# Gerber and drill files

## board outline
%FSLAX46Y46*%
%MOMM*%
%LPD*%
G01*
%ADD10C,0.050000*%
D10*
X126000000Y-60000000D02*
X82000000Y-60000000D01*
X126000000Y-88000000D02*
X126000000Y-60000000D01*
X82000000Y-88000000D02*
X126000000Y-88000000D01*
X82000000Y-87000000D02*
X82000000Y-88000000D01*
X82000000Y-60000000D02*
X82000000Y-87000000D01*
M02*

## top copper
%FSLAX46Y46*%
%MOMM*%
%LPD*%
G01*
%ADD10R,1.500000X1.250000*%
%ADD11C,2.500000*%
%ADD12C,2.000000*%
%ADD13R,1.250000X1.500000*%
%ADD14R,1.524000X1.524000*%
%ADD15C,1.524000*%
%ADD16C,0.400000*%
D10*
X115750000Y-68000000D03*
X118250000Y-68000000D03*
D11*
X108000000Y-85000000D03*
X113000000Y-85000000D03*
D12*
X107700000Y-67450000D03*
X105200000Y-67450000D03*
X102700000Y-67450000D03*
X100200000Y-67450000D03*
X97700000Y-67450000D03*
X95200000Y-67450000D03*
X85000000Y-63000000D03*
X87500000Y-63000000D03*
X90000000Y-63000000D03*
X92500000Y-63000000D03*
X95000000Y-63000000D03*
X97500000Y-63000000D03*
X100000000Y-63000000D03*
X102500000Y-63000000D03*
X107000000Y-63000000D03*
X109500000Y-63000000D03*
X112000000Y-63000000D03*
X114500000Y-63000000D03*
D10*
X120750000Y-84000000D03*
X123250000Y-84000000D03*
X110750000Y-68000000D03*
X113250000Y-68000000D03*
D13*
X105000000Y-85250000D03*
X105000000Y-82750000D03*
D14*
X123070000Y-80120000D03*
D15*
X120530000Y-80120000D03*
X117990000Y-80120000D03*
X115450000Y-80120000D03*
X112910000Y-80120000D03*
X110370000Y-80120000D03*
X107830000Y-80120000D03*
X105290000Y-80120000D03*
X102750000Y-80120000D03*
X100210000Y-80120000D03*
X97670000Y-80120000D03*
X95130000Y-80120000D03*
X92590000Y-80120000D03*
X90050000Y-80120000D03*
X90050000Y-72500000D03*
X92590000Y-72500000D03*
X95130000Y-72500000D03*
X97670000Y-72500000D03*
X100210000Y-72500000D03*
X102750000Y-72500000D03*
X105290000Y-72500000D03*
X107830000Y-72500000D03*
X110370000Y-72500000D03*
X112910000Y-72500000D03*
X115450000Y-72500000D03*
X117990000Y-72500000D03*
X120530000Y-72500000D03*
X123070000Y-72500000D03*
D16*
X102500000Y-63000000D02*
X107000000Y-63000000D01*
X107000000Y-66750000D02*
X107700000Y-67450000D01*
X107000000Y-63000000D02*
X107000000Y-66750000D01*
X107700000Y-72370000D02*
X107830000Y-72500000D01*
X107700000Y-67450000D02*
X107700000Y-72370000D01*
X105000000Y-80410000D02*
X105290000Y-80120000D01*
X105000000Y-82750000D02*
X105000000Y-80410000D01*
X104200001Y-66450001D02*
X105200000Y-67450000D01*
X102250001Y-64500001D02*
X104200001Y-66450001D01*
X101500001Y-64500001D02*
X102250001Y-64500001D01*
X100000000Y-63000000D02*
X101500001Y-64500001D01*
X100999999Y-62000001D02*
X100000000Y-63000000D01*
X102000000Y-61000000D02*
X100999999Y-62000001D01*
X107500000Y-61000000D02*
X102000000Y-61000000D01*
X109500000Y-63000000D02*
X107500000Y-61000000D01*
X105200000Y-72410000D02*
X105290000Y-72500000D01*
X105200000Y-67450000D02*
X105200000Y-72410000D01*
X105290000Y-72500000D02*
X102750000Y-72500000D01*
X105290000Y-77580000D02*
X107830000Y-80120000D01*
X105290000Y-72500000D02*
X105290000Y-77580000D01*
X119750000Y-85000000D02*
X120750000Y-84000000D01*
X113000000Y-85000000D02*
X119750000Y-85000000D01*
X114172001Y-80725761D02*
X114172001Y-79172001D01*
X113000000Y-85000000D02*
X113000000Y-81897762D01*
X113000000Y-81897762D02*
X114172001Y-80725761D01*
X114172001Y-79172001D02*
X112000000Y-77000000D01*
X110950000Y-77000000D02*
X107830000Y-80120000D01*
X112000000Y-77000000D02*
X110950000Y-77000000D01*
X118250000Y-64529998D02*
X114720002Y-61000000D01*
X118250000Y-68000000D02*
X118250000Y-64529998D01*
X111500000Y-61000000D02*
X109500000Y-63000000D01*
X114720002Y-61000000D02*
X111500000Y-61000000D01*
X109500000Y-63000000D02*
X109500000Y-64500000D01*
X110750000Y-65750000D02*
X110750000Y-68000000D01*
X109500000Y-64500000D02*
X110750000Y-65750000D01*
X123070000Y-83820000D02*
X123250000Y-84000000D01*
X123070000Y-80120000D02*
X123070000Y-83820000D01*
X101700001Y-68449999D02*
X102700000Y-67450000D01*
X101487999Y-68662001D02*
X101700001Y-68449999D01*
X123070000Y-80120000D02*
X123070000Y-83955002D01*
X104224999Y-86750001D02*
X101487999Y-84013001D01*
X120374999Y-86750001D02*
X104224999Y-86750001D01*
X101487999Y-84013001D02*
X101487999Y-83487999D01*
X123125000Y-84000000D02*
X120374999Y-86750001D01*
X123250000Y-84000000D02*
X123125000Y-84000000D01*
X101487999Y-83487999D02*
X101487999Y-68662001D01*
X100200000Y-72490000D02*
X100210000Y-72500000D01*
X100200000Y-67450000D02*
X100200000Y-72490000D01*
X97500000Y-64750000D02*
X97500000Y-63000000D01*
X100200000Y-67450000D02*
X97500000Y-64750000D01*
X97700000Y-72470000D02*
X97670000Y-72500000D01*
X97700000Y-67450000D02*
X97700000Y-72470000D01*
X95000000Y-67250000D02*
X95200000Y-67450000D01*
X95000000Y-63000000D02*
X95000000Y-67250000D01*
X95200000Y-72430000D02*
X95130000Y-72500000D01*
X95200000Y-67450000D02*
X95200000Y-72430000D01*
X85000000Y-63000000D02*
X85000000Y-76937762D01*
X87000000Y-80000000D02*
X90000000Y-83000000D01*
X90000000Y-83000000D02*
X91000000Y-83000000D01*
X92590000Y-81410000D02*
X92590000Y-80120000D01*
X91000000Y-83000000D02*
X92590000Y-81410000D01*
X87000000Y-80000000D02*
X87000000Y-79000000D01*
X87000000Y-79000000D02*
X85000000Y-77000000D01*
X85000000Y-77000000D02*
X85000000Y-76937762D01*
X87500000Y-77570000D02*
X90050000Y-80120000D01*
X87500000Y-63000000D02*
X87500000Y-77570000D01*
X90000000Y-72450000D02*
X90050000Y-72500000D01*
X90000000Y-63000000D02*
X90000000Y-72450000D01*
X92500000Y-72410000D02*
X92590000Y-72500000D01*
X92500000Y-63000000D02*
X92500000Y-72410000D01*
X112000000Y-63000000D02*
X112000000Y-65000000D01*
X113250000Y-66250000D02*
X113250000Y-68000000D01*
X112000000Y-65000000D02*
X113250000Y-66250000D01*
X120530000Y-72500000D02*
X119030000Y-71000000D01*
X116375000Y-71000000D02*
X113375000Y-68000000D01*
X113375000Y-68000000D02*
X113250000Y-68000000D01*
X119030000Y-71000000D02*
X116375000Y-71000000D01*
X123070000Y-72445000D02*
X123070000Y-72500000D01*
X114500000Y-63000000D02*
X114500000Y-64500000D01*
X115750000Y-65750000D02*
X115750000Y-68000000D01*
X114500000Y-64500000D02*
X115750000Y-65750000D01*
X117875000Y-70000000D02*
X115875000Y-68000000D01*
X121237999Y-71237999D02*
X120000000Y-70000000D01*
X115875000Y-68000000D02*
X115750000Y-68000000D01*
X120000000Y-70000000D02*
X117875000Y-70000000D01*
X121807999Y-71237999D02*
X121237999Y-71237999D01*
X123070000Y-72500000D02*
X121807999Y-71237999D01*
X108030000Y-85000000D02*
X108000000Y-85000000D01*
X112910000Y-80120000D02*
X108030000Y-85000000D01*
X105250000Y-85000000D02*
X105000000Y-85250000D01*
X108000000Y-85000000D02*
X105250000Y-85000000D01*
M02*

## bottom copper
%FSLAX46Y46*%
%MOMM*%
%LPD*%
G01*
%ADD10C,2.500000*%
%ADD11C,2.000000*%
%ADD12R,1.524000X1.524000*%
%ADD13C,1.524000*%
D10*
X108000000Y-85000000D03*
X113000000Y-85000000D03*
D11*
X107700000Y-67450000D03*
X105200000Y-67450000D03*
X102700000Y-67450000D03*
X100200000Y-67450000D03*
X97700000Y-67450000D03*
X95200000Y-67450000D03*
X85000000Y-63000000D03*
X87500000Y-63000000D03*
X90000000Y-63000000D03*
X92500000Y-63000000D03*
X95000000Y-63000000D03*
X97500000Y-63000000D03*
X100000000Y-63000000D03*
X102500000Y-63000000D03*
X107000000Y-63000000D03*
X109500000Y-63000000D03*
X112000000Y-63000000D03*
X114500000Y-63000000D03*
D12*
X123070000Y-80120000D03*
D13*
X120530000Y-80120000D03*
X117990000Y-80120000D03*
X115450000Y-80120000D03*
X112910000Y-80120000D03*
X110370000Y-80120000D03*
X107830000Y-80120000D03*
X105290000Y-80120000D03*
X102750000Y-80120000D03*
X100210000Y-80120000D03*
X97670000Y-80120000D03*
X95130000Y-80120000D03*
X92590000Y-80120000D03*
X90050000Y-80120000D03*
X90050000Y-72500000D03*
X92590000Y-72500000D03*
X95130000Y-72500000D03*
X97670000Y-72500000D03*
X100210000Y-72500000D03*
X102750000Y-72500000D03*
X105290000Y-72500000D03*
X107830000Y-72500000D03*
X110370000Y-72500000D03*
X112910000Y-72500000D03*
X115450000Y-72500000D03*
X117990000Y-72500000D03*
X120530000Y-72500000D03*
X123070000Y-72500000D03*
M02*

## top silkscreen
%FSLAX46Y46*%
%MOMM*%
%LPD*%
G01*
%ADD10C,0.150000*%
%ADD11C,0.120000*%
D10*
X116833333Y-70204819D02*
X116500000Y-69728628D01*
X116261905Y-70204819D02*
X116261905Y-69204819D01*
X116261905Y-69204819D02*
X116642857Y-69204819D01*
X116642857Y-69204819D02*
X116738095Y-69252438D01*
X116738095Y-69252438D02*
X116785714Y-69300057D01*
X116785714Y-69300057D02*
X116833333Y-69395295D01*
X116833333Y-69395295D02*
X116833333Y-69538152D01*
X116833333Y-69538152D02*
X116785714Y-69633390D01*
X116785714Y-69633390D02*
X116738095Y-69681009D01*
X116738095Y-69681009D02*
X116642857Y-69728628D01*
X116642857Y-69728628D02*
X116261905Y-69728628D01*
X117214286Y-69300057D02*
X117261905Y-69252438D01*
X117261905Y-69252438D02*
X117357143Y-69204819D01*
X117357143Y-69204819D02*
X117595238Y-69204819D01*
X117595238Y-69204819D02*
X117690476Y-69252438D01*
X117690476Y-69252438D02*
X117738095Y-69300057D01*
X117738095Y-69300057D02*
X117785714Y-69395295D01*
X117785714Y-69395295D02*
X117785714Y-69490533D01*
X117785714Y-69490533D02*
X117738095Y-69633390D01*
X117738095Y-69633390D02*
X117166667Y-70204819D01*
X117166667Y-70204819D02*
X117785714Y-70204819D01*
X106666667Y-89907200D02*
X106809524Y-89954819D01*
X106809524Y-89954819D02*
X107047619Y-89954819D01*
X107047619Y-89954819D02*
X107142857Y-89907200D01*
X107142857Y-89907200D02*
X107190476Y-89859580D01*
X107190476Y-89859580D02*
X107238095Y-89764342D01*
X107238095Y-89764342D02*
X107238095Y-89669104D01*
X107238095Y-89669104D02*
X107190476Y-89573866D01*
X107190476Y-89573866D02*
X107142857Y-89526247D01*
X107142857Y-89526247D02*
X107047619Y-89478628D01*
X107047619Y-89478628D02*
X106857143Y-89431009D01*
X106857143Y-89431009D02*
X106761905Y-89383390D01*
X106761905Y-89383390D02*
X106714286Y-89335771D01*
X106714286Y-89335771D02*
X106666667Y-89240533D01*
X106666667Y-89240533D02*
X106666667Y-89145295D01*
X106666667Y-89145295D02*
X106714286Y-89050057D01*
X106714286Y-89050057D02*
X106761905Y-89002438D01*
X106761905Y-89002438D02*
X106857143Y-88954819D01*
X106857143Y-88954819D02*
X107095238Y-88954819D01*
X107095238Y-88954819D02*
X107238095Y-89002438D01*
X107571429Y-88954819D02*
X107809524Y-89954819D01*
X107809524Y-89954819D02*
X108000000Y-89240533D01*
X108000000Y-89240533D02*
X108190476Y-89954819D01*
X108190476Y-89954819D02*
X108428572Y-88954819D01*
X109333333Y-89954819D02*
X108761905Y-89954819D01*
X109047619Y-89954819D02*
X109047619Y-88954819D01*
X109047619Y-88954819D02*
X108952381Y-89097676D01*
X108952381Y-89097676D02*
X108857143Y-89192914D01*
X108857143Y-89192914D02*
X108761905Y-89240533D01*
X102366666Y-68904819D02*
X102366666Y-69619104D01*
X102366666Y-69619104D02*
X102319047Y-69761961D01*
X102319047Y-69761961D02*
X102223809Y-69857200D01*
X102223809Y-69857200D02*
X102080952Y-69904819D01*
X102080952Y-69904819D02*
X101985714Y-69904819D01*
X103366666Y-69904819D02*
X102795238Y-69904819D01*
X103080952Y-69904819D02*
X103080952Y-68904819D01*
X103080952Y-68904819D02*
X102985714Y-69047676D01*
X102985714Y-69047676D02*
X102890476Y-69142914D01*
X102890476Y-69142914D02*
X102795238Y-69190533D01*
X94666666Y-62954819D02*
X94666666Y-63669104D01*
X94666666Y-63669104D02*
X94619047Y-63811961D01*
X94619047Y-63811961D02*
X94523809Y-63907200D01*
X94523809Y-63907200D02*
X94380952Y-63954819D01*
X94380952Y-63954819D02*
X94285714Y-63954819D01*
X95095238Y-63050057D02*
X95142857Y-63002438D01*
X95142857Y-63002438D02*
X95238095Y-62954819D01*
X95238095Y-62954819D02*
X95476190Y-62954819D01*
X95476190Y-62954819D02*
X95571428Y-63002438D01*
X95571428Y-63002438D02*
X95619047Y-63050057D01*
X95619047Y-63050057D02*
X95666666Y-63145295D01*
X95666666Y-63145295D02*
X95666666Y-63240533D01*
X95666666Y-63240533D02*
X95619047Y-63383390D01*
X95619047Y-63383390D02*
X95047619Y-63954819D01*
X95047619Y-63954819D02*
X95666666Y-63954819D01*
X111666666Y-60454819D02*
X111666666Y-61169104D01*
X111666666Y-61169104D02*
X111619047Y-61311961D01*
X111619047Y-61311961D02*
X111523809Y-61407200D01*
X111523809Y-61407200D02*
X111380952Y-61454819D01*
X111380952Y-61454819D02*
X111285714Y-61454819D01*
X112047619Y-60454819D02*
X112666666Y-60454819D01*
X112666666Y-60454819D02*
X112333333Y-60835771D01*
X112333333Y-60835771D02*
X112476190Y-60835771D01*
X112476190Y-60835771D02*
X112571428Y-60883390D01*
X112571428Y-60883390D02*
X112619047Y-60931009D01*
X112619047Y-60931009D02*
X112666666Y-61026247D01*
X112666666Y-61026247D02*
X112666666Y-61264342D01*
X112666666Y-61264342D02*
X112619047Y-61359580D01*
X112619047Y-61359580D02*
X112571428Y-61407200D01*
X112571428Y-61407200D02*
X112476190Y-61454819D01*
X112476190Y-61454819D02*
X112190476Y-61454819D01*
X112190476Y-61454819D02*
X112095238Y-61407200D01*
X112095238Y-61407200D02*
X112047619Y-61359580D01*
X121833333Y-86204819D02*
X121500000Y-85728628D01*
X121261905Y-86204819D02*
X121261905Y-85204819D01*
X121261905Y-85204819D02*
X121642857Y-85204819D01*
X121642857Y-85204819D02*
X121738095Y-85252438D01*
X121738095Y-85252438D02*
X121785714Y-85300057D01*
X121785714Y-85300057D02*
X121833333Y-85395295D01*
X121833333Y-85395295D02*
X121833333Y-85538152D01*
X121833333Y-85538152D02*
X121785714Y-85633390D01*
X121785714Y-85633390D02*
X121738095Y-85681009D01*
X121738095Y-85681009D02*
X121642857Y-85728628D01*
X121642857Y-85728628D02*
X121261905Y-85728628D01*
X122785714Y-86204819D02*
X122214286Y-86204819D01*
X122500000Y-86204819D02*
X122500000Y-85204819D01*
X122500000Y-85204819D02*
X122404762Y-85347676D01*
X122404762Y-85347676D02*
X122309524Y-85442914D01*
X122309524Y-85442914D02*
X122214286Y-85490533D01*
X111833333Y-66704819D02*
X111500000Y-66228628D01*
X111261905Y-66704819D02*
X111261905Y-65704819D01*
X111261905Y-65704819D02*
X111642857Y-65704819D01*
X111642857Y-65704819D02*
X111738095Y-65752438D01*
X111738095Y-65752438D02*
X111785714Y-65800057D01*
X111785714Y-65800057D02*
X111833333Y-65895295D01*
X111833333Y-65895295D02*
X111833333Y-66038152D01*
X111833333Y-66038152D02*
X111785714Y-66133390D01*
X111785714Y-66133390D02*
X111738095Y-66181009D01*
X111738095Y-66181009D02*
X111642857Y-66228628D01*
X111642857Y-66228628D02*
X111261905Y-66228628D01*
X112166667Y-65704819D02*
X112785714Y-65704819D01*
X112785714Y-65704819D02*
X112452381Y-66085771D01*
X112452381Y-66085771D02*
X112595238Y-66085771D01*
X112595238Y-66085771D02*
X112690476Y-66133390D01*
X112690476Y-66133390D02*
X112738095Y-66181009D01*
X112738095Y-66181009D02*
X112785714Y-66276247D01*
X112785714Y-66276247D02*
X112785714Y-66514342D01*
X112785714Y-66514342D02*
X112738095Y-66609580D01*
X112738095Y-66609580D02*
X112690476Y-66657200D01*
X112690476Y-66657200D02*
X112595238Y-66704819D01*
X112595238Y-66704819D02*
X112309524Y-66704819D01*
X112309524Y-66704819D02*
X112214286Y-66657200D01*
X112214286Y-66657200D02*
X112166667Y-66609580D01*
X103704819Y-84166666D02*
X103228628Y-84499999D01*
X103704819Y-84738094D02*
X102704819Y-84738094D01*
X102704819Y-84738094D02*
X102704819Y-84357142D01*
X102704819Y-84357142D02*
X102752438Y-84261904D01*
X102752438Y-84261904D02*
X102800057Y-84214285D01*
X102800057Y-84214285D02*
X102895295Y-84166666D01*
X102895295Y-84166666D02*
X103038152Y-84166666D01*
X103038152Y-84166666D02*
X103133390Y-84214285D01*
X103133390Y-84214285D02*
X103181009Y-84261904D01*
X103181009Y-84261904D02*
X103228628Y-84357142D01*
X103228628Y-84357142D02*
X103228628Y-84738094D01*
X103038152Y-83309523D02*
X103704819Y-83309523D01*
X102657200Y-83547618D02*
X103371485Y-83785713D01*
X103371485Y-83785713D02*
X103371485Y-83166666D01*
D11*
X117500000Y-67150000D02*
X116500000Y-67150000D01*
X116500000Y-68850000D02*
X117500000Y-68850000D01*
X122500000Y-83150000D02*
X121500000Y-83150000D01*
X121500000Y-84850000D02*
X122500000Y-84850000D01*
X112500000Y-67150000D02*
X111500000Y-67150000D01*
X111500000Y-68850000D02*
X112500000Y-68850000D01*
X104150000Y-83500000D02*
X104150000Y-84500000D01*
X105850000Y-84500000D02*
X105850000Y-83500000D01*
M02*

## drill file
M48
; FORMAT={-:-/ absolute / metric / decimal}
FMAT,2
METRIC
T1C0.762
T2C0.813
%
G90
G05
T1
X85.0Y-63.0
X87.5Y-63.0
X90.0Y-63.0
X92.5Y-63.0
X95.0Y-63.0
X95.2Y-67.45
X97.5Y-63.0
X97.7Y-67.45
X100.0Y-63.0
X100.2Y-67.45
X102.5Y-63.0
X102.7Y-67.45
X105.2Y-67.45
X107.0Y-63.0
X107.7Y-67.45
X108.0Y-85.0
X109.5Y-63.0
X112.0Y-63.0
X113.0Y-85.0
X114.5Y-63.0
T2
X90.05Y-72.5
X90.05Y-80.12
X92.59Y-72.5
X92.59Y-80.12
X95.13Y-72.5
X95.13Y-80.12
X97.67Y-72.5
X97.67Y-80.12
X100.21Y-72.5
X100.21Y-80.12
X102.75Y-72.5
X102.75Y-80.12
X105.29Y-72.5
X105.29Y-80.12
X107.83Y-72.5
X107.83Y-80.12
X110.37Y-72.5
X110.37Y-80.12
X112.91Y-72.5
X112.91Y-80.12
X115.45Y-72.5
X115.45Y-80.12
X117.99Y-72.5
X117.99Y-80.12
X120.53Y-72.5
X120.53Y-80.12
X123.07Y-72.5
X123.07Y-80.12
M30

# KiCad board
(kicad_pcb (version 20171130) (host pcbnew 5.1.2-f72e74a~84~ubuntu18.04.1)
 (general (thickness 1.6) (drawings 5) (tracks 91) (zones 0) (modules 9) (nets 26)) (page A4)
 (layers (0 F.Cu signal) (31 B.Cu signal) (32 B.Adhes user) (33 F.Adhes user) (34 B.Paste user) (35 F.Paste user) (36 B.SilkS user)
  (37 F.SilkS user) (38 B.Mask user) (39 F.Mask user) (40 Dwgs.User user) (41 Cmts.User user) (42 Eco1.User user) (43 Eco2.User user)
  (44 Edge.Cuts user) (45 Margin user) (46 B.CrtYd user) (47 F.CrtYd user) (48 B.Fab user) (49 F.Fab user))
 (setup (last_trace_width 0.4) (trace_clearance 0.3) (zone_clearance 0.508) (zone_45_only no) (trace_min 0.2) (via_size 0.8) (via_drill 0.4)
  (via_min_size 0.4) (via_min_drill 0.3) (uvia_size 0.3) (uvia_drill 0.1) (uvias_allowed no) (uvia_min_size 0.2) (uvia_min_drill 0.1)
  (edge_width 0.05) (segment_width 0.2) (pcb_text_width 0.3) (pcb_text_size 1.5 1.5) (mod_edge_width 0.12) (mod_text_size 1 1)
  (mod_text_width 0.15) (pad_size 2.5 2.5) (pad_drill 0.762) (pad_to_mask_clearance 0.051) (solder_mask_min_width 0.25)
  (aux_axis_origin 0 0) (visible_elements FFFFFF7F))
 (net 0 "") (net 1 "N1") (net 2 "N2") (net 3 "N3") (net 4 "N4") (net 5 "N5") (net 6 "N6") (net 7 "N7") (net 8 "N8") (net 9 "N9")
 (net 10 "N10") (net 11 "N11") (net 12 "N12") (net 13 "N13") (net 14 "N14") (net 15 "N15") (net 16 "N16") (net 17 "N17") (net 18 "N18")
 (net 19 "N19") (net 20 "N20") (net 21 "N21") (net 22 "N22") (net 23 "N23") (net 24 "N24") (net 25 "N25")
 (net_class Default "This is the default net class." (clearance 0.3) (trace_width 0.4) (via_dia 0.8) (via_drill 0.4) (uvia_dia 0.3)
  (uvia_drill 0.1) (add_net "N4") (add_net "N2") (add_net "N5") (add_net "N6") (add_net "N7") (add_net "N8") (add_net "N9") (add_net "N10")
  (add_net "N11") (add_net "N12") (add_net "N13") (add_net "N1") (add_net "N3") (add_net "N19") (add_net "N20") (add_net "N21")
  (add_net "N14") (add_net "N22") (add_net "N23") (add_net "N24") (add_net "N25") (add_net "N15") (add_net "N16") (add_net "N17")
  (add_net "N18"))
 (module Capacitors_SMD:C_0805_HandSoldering (layer F.Cu) (at 117 68 180)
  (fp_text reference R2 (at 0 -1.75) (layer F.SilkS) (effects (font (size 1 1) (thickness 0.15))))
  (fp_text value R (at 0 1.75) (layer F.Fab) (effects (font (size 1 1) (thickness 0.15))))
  (fp_line (start -0.5 0.85) (end 0.5 0.85) (layer F.SilkS) (width 0.12))
  (fp_line (start 0.5 -0.85) (end -0.5 -0.85) (layer F.SilkS) (width 0.12))
  (pad 2 smd rect (at 1.25 0 180) (size 1.5 1.25) (layers F.Cu F.Paste F.Mask) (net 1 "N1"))
  (pad 1 smd rect (at -1.25 0 180) (size 1.5 1.25) (layers F.Cu F.Paste F.Mask) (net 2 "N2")))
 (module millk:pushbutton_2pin (layer F.Cu) (at 108 90 180)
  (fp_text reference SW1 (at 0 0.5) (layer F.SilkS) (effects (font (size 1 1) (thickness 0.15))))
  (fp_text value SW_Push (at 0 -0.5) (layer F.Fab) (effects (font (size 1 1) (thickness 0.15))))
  (pad 2 thru_hole circle (at 0 5 180) (size 2.5 2.5) (drill 0.762) (layers *.Cu *.Mask) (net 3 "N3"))
  (pad 1 thru_hole circle (at -5 5 180) (size 2.5 2.5) (drill 0.762) (layers *.Cu *.Mask) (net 2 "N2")))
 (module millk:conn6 (layer F.Cu) (at 102.7 69.95 180)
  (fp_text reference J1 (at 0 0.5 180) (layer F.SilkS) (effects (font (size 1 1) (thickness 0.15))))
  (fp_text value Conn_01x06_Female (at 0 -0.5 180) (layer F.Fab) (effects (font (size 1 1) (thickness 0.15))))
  (pad 1 thru_hole circle (at -5 2.5 180) (size 2 2) (drill 0.762) (layers *.Cu *.Mask) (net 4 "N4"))
  (pad 2 thru_hole circle (at -2.5 2.5 180) (size 2 2) (drill 0.762) (layers *.Cu *.Mask) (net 2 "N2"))
  (pad 3 thru_hole circle (at 0 2.5 180) (size 2 2) (drill 0.762) (layers *.Cu *.Mask) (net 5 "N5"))
  (pad 4 thru_hole circle (at 2.5 2.5 180) (size 2 2) (drill 0.762) (layers *.Cu *.Mask) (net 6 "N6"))
  (pad 5 thru_hole circle (at 5 2.5 180) (size 2 2) (drill 0.762) (layers *.Cu *.Mask) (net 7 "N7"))
  (pad 6 thru_hole circle (at 7.5 2.5 180) (size 2 2) (drill 0.762) (layers *.Cu *.Mask) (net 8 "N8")))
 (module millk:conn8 (layer F.Cu) (at 95 63)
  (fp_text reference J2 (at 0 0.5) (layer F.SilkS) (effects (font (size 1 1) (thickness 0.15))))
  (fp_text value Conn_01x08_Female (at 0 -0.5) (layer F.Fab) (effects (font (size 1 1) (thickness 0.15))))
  (pad 1 thru_hole circle (at -10 0) (size 2 2) (drill 0.762) (layers *.Cu *.Mask) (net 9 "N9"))
  (pad 2 thru_hole circle (at -7.5 0) (size 2 2) (drill 0.762) (layers *.Cu *.Mask) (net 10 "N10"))
  (pad 3 thru_hole circle (at -5 0) (size 2 2) (drill 0.762) (layers *.Cu *.Mask) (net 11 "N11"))
  (pad 4 thru_hole circle (at -2.5 0) (size 2 2) (drill 0.762) (layers *.Cu *.Mask) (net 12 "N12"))
  (pad 5 thru_hole circle (at 0 0) (size 2 2) (drill 0.762) (layers *.Cu *.Mask) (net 8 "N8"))
  (pad 6 thru_hole circle (at 2.5 0) (size 2 2) (drill 0.762) (layers *.Cu *.Mask) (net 6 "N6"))
  (pad 7 thru_hole circle (at 5 0) (size 2 2) (drill 0.762) (layers *.Cu *.Mask) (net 2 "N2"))
  (pad 8 thru_hole circle (at 7.5 0) (size 2 2) (drill 0.762) (layers *.Cu *.Mask) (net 4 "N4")))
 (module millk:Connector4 (layer F.Cu) (at 112 60.5)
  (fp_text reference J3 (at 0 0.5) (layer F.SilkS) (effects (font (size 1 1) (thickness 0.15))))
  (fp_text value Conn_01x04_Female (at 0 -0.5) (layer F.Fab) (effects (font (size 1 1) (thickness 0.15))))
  (pad 1 thru_hole circle (at -5 2.5) (size 2 2) (drill 0.762) (layers *.Cu *.Mask) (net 4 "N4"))
  (pad 2 thru_hole circle (at -2.5 2.5) (size 2 2) (drill 0.762) (layers *.Cu *.Mask) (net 2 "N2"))
  (pad 3 thru_hole circle (at 0 2.5) (size 2 2) (drill 0.762) (layers *.Cu *.Mask) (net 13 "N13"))
  (pad 4 thru_hole circle (at 2.5 2.5) (size 2 2) (drill 0.762) (layers *.Cu *.Mask) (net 1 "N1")))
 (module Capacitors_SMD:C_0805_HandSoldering (layer F.Cu) (at 122 84 180)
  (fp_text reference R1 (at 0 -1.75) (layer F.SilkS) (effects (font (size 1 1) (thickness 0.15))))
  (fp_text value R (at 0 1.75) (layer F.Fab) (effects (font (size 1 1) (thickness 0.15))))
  (fp_line (start -0.5 0.85) (end 0.5 0.85) (layer F.SilkS) (width 0.12))
  (fp_line (start 0.5 -0.85) (end -0.5 -0.85) (layer F.SilkS) (width 0.12))
  (pad 2 smd rect (at 1.25 0 180) (size 1.5 1.25) (layers F.Cu F.Paste F.Mask) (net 2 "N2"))
  (pad 1 smd rect (at -1.25 0 180) (size 1.5 1.25) (layers F.Cu F.Paste F.Mask) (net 5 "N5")))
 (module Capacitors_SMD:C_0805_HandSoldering (layer F.Cu) (at 112 68)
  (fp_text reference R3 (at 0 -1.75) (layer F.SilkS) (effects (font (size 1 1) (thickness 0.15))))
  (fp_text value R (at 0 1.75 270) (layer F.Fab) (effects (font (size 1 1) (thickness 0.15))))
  (fp_line (start 0.5 -0.85) (end -0.5 -0.85) (layer F.SilkS) (width 0.12))
  (fp_line (start -0.5 0.85) (end 0.5 0.85) (layer F.SilkS) (width 0.12))
  (pad 1 smd rect (at -1.25 0) (size 1.5 1.25) (layers F.Cu F.Paste F.Mask) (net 2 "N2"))
  (pad 2 smd rect (at 1.25 0) (size 1.5 1.25) (layers F.Cu F.Paste F.Mask) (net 13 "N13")))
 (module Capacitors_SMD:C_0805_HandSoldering (layer F.Cu) (at 105 84 90)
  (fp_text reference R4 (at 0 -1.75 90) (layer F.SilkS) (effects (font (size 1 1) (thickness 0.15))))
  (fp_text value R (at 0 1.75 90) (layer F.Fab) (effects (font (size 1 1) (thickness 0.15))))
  (fp_line (start 0.5 -0.85) (end -0.5 -0.85) (layer F.SilkS) (width 0.12))
  (fp_line (start -0.5 0.85) (end 0.5 0.85) (layer F.SilkS) (width 0.12))
  (pad 1 smd rect (at -1.25 0 90) (size 1.5 1.25) (layers F.Cu F.Paste F.Mask) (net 3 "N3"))
  (pad 2 smd rect (at 1.25 0 90) (size 1.5 1.25) (layers F.Cu F.Paste F.Mask) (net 4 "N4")))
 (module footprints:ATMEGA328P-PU (layer B.Cu) (at 90.05 72.5 90)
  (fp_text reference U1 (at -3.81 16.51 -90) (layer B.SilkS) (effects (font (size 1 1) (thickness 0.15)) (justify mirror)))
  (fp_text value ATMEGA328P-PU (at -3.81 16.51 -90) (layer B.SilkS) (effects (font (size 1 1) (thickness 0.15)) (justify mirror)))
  (pad 1 thru_hole rect (at -7.62 33.02 90) (size 1.524 1.524) (drill 0.8128) (layers *.Cu *.Mask) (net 5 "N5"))
  (pad 2 thru_hole circle (at -7.62 30.48 90) (size 1.524 1.524) (drill 0.8128) (layers *.Cu *.Mask) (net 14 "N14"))
  (pad 3 thru_hole circle (at -7.62 27.94 90) (size 1.524 1.524) (drill 0.8128) (layers *.Cu *.Mask) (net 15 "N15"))
  (pad 4 thru_hole circle (at -7.62 25.4 90) (size 1.524 1.524) (drill 0.8128) (layers *.Cu *.Mask) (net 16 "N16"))
  (pad 5 thru_hole circle (at -7.62 22.86 90) (size 1.524 1.524) (drill 0.8128) (layers *.Cu *.Mask) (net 3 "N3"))
  (pad 6 thru_hole circle (at -7.62 20.32 90) (size 1.524 1.524) (drill 0.8128) (layers *.Cu *.Mask) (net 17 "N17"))
  (pad 7 thru_hole circle (at -7.62 17.78 90) (size 1.524 1.524) (drill 0.8128) (layers *.Cu *.Mask) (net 2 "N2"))
  (pad 8 thru_hole circle (at -7.62 15.24 90) (size 1.524 1.524) (drill 0.8128) (layers *.Cu *.Mask) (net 4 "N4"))
  (pad 9 thru_hole circle (at -7.62 12.7 90) (size 1.524 1.524) (drill 0.8128) (layers *.Cu *.Mask) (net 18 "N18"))
  (pad 10 thru_hole circle (at -7.62 10.16 90) (size 1.524 1.524) (drill 0.8128) (layers *.Cu *.Mask) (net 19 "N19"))
  (pad 11 thru_hole circle (at -7.62 7.62 90) (size 1.524 1.524) (drill 0.8128) (layers *.Cu *.Mask) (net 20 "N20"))
  (pad 12 thru_hole circle (at -7.62 5.08 90) (size 1.524 1.524) (drill 0.8128) (layers *.Cu *.Mask) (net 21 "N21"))
  (pad 13 thru_hole circle (at -7.62 2.54 90) (size 1.524 1.524) (drill 0.8128) (layers *.Cu *.Mask) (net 9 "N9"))
  (pad 14 thru_hole circle (at -7.62 0 90) (size 1.524 1.524) (drill 0.8128) (layers *.Cu *.Mask) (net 10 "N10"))
  (pad 15 thru_hole circle (at 0 0 90) (size 1.524 1.524) (drill 0.8128) (layers *.Cu *.Mask) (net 11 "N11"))
  (pad 16 thru_hole circle (at 0 2.54 90) (size 1.524 1.524) (drill 0.8128) (layers *.Cu *.Mask) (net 12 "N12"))
  (pad 17 thru_hole circle (at 0 5.08 90) (size 1.524 1.524) (drill 0.8128) (layers *.Cu *.Mask) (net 8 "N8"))
  (pad 18 thru_hole circle (at 0 7.62 90) (size 1.524 1.524) (drill 0.8128) (layers *.Cu *.Mask) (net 7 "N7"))
  (pad 19 thru_hole circle (at 0 10.16 90) (size 1.524 1.524) (drill 0.8128) (layers *.Cu *.Mask) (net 6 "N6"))
  (pad 20 thru_hole circle (at 0 12.7 90) (size 1.524 1.524) (drill 0.8128) (layers *.Cu *.Mask) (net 2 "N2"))
  (pad 21 thru_hole circle (at 0 15.24 90) (size 1.524 1.524) (drill 0.8128) (layers *.Cu *.Mask) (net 2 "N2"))
  (pad 22 thru_hole circle (at 0 17.78 90) (size 1.524 1.524) (drill 0.8128) (layers *.Cu *.Mask) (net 4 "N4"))
  (pad 23 thru_hole circle (at 0 20.32 90) (size 1.524 1.524) (drill 0.8128) (layers *.Cu *.Mask) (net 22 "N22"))
  (pad 24 thru_hole circle (at 0 22.86 90) (size 1.524 1.524) (drill 0.8128) (layers *.Cu *.Mask) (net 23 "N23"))
  (pad 25 thru_hole circle (at 0 25.4 90) (size 1.524 1.524) (drill 0.8128) (layers *.Cu *.Mask) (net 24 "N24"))
  (pad 26 thru_hole circle (at 0 27.94 90) (size 1.524 1.524) (drill 0.8128) (layers *.Cu *.Mask) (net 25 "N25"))
  (pad 27 thru_hole circle (at 0 30.48 90) (size 1.524 1.524) (drill 0.8128) (layers *.Cu *.Mask) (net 13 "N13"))
  (pad 28 thru_hole circle (at 0 33.02 90) (size 1.524 1.524) (drill 0.8128) (layers *.Cu *.Mask) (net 1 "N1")))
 (gr_line (start 126 60) (end 82 60) (layer Edge.Cuts) (width 0.05))
 (gr_line (start 126 88) (end 126 60) (layer Edge.Cuts) (width 0.05))
 (gr_line (start 82 88) (end 126 88) (layer Edge.Cuts) (width 0.05))
 (gr_line (start 82 87) (end 82 88) (layer Edge.Cuts) (width 0.05))
 (gr_line (start 82 60) (end 82 87) (layer Edge.Cuts) (width 0.05))
 (segment (start 102.5 63) (end 107 63) (width 0.4) (layer F.Cu) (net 4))
 (segment (start 107 66.75) (end 107.7 67.45) (width 0.4) (layer F.Cu) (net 4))
 (segment (start 107 63) (end 107 66.75) (width 0.4) (layer F.Cu) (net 4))
 (segment (start 107.7 72.37) (end 107.83 72.5) (width 0.4) (layer F.Cu) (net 4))
 (segment (start 107.7 67.45) (end 107.7 72.37) (width 0.4) (layer F.Cu) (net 4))
 (segment (start 105 80.41) (end 105.29 80.12) (width 0.4) (layer F.Cu) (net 4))
 (segment (start 105 82.75) (end 105 80.41) (width 0.4) (layer F.Cu) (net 4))
 (segment (start 104.200001 66.450001) (end 105.2 67.45) (width 0.4) (layer F.Cu) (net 2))
 (segment (start 102.250001 64.500001) (end 104.200001 66.450001) (width 0.4) (layer F.Cu) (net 2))
 (segment (start 101.500001 64.500001) (end 102.250001 64.500001) (width 0.4) (layer F.Cu) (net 2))
 (segment (start 100 63) (end 101.500001 64.500001) (width 0.4) (layer F.Cu) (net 2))
 (segment (start 100.999999 62.000001) (end 100 63) (width 0.4) (layer F.Cu) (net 2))
 (segment (start 102 61) (end 100.999999 62.000001) (width 0.4) (layer F.Cu) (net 2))
 (segment (start 107.5 61) (end 102 61) (width 0.4) (layer F.Cu) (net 2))
 (segment (start 109.5 63) (end 107.5 61) (width 0.4) (layer F.Cu) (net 2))
 (segment (start 105.2 72.41) (end 105.29 72.5) (width 0.4) (layer F.Cu) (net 2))
 (segment (start 105.2 67.45) (end 105.2 72.41) (width 0.4) (layer F.Cu) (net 2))
 (segment (start 105.29 72.5) (end 102.75 72.5) (width 0.4) (layer F.Cu) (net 2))
 (segment (start 105.29 77.58) (end 107.83 80.12) (width 0.4) (layer F.Cu) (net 2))
 (segment (start 105.29 72.5) (end 105.29 77.58) (width 0.4) (layer F.Cu) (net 2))
 (segment (start 119.75 85) (end 120.75 84) (width 0.4) (layer F.Cu) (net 2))
 (segment (start 113 85) (end 119.75 85) (width 0.4) (layer F.Cu) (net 2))
 (segment (start 114.172001 80.725761) (end 114.172001 79.172001) (width 0.4) (layer F.Cu) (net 2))
 (segment (start 113 85) (end 113 81.897762) (width 0.4) (layer F.Cu) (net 2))
 (segment (start 113 81.897762) (end 114.172001 80.725761) (width 0.4) (layer F.Cu) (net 2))
 (segment (start 114.172001 79.172001) (end 112 77) (width 0.4) (layer F.Cu) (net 2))
 (segment (start 110.95 77) (end 107.83 80.12) (width 0.4) (layer F.Cu) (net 2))
 (segment (start 112 77) (end 110.95 77) (width 0.4) (layer F.Cu) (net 2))
 (segment (start 118.25 64.529998) (end 114.720002 61) (width 0.4) (layer F.Cu) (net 2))
 (segment (start 118.25 68) (end 118.25 64.529998) (width 0.4) (layer F.Cu) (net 2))
 (segment (start 111.5 61) (end 109.5 63) (width 0.4) (layer F.Cu) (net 2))
 (segment (start 114.720002 61) (end 111.5 61) (width 0.4) (layer F.Cu) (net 2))
 (segment (start 109.5 63) (end 109.5 64.5) (width 0.4) (layer F.Cu) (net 2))
 (segment (start 110.75 65.75) (end 110.75 68) (width 0.4) (layer F.Cu) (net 2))
 (segment (start 109.5 64.5) (end 110.75 65.75) (width 0.4) (layer F.Cu) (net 2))
 (segment (start 123.07 83.82) (end 123.25 84) (width 0.4) (layer F.Cu) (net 5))
 (segment (start 123.07 80.12) (end 123.07 83.82) (width 0.4) (layer F.Cu) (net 5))
 (segment (start 101.700001 68.449999) (end 102.7 67.45) (width 0.4) (layer F.Cu) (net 5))
 (segment (start 101.487999 68.662001) (end 101.700001 68.449999) (width 0.4) (layer F.Cu) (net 5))
 (segment (start 123.07 80.12) (end 123.07 83.955002) (width 0.4) (layer F.Cu) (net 5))
 (segment (start 104.224999 86.750001) (end 101.487999 84.013001) (width 0.4) (layer F.Cu) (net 5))
 (segment (start 120.374999 86.750001) (end 104.224999 86.750001) (width 0.4) (layer F.Cu) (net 5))
 (segment (start 101.487999 84.013001) (end 101.487999 83.487999) (width 0.4) (layer F.Cu) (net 5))
 (segment (start 123.125 84) (end 120.374999 86.750001) (width 0.4) (layer F.Cu) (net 5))
 (segment (start 123.25 84) (end 123.125 84) (width 0.4) (layer F.Cu) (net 5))
 (segment (start 101.487999 83.487999) (end 101.487999 68.662001) (width 0.4) (layer F.Cu) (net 5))
 (segment (start 100.2 72.49) (end 100.21 72.5) (width 0.4) (layer F.Cu) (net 6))
 (segment (start 100.2 67.45) (end 100.2 72.49) (width 0.4) (layer F.Cu) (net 6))
 (segment (start 97.5 64.75) (end 97.5 63) (width 0.4) (layer F.Cu) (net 6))
 (segment (start 100.2 67.45) (end 97.5 64.75) (width 0.4) (layer F.Cu) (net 6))
 (segment (start 97.7 72.47) (end 97.67 72.5) (width 0.4) (layer F.Cu) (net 7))
 (segment (start 97.7 67.45) (end 97.7 72.47) (width 0.4) (layer F.Cu) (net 7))
 (segment (start 95 67.25) (end 95.2 67.45) (width 0.4) (layer F.Cu) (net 8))
 (segment (start 95 63) (end 95 67.25) (width 0.4) (layer F.Cu) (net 8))
 (segment (start 95.2 72.43) (end 95.13 72.5) (width 0.4) (layer F.Cu) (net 8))
 (segment (start 95.2 67.45) (end 95.2 72.43) (width 0.4) (layer F.Cu) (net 8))
 (segment (start 85 63) (end 85 76.937762) (width 0.4) (layer F.Cu) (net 9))
 (segment (start 87 80) (end 90 83) (width 0.4) (layer F.Cu) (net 9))
 (segment (start 90 83) (end 91 83) (width 0.4) (layer F.Cu) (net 9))
 (segment (start 92.59 81.41) (end 92.59 80.12) (width 0.4) (layer F.Cu) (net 9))
 (segment (start 91 83) (end 92.59 81.41) (width 0.4) (layer F.Cu) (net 9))
 (segment (start 87 80) (end 87 79) (width 0.4) (layer F.Cu) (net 9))
 (segment (start 87 79) (end 85 77) (width 0.4) (layer F.Cu) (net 9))
 (segment (start 85 77) (end 85 76.937762) (width 0.4) (layer F.Cu) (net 9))
 (segment (start 87.5 77.57) (end 90.05 80.12) (width 0.4) (layer F.Cu) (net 10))
 (segment (start 87.5 63) (end 87.5 77.57) (width 0.4) (layer F.Cu) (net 10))
 (segment (start 90 72.45) (end 90.05 72.5) (width 0.4) (layer F.Cu) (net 11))
 (segment (start 90 63) (end 90 72.45) (width 0.4) (layer F.Cu) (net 11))
 (segment (start 92.5 72.41) (end 92.59 72.5) (width 0.4) (layer F.Cu) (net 12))
 (segment (start 92.5 63) (end 92.5 72.41) (width 0.4) (layer F.Cu) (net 12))
 (segment (start 112 63) (end 112 65) (width 0.4) (layer F.Cu) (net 13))
 (segment (start 113.25 66.25) (end 113.25 68) (width 0.4) (layer F.Cu) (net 13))
 (segment (start 112 65) (end 113.25 66.25) (width 0.4) (layer F.Cu) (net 13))
 (segment (start 120.53 72.5) (end 119.03 71) (width 0.4) (layer F.Cu) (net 13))
 (segment (start 116.375 71) (end 113.375 68) (width 0.4) (layer F.Cu) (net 13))
 (segment (start 113.375 68) (end 113.25 68) (width 0.4) (layer F.Cu) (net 13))
 (segment (start 119.03 71) (end 116.375 71) (width 0.4) (layer F.Cu) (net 13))
 (segment (start 123.07 72.445) (end 123.07 72.5) (width 0.4) (layer F.Cu) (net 1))
 (segment (start 114.5 63) (end 114.5 64.5) (width 0.4) (layer F.Cu) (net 1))
 (segment (start 115.75 65.75) (end 115.75 68) (width 0.4) (layer F.Cu) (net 1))
 (segment (start 114.5 64.5) (end 115.75 65.75) (width 0.4) (layer F.Cu) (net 1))
 (segment (start 117.875 70) (end 115.875 68) (width 0.4) (layer F.Cu) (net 1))
 (segment (start 121.237999 71.237999) (end 120 70) (width 0.4) (layer F.Cu) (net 1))
 (segment (start 115.875 68) (end 115.75 68) (width 0.4) (layer F.Cu) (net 1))
 (segment (start 120 70) (end 117.875 70) (width 0.4) (layer F.Cu) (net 1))
 (segment (start 121.807999 71.237999) (end 121.237999 71.237999) (width 0.4) (layer F.Cu) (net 1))
 (segment (start 123.07 72.5) (end 121.807999 71.237999) (width 0.4) (layer F.Cu) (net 1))
 (segment (start 108.03 85) (end 108 85) (width 0.4) (layer F.Cu) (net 3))
 (segment (start 112.91 80.12) (end 108.03 85) (width 0.4) (layer F.Cu) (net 3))
 (segment (start 105.25 85) (end 105 85.25) (width 0.4) (layer F.Cu) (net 3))
 (segment (start 108 85) (end 105.25 85) (width 0.4) (layer F.Cu) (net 3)))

